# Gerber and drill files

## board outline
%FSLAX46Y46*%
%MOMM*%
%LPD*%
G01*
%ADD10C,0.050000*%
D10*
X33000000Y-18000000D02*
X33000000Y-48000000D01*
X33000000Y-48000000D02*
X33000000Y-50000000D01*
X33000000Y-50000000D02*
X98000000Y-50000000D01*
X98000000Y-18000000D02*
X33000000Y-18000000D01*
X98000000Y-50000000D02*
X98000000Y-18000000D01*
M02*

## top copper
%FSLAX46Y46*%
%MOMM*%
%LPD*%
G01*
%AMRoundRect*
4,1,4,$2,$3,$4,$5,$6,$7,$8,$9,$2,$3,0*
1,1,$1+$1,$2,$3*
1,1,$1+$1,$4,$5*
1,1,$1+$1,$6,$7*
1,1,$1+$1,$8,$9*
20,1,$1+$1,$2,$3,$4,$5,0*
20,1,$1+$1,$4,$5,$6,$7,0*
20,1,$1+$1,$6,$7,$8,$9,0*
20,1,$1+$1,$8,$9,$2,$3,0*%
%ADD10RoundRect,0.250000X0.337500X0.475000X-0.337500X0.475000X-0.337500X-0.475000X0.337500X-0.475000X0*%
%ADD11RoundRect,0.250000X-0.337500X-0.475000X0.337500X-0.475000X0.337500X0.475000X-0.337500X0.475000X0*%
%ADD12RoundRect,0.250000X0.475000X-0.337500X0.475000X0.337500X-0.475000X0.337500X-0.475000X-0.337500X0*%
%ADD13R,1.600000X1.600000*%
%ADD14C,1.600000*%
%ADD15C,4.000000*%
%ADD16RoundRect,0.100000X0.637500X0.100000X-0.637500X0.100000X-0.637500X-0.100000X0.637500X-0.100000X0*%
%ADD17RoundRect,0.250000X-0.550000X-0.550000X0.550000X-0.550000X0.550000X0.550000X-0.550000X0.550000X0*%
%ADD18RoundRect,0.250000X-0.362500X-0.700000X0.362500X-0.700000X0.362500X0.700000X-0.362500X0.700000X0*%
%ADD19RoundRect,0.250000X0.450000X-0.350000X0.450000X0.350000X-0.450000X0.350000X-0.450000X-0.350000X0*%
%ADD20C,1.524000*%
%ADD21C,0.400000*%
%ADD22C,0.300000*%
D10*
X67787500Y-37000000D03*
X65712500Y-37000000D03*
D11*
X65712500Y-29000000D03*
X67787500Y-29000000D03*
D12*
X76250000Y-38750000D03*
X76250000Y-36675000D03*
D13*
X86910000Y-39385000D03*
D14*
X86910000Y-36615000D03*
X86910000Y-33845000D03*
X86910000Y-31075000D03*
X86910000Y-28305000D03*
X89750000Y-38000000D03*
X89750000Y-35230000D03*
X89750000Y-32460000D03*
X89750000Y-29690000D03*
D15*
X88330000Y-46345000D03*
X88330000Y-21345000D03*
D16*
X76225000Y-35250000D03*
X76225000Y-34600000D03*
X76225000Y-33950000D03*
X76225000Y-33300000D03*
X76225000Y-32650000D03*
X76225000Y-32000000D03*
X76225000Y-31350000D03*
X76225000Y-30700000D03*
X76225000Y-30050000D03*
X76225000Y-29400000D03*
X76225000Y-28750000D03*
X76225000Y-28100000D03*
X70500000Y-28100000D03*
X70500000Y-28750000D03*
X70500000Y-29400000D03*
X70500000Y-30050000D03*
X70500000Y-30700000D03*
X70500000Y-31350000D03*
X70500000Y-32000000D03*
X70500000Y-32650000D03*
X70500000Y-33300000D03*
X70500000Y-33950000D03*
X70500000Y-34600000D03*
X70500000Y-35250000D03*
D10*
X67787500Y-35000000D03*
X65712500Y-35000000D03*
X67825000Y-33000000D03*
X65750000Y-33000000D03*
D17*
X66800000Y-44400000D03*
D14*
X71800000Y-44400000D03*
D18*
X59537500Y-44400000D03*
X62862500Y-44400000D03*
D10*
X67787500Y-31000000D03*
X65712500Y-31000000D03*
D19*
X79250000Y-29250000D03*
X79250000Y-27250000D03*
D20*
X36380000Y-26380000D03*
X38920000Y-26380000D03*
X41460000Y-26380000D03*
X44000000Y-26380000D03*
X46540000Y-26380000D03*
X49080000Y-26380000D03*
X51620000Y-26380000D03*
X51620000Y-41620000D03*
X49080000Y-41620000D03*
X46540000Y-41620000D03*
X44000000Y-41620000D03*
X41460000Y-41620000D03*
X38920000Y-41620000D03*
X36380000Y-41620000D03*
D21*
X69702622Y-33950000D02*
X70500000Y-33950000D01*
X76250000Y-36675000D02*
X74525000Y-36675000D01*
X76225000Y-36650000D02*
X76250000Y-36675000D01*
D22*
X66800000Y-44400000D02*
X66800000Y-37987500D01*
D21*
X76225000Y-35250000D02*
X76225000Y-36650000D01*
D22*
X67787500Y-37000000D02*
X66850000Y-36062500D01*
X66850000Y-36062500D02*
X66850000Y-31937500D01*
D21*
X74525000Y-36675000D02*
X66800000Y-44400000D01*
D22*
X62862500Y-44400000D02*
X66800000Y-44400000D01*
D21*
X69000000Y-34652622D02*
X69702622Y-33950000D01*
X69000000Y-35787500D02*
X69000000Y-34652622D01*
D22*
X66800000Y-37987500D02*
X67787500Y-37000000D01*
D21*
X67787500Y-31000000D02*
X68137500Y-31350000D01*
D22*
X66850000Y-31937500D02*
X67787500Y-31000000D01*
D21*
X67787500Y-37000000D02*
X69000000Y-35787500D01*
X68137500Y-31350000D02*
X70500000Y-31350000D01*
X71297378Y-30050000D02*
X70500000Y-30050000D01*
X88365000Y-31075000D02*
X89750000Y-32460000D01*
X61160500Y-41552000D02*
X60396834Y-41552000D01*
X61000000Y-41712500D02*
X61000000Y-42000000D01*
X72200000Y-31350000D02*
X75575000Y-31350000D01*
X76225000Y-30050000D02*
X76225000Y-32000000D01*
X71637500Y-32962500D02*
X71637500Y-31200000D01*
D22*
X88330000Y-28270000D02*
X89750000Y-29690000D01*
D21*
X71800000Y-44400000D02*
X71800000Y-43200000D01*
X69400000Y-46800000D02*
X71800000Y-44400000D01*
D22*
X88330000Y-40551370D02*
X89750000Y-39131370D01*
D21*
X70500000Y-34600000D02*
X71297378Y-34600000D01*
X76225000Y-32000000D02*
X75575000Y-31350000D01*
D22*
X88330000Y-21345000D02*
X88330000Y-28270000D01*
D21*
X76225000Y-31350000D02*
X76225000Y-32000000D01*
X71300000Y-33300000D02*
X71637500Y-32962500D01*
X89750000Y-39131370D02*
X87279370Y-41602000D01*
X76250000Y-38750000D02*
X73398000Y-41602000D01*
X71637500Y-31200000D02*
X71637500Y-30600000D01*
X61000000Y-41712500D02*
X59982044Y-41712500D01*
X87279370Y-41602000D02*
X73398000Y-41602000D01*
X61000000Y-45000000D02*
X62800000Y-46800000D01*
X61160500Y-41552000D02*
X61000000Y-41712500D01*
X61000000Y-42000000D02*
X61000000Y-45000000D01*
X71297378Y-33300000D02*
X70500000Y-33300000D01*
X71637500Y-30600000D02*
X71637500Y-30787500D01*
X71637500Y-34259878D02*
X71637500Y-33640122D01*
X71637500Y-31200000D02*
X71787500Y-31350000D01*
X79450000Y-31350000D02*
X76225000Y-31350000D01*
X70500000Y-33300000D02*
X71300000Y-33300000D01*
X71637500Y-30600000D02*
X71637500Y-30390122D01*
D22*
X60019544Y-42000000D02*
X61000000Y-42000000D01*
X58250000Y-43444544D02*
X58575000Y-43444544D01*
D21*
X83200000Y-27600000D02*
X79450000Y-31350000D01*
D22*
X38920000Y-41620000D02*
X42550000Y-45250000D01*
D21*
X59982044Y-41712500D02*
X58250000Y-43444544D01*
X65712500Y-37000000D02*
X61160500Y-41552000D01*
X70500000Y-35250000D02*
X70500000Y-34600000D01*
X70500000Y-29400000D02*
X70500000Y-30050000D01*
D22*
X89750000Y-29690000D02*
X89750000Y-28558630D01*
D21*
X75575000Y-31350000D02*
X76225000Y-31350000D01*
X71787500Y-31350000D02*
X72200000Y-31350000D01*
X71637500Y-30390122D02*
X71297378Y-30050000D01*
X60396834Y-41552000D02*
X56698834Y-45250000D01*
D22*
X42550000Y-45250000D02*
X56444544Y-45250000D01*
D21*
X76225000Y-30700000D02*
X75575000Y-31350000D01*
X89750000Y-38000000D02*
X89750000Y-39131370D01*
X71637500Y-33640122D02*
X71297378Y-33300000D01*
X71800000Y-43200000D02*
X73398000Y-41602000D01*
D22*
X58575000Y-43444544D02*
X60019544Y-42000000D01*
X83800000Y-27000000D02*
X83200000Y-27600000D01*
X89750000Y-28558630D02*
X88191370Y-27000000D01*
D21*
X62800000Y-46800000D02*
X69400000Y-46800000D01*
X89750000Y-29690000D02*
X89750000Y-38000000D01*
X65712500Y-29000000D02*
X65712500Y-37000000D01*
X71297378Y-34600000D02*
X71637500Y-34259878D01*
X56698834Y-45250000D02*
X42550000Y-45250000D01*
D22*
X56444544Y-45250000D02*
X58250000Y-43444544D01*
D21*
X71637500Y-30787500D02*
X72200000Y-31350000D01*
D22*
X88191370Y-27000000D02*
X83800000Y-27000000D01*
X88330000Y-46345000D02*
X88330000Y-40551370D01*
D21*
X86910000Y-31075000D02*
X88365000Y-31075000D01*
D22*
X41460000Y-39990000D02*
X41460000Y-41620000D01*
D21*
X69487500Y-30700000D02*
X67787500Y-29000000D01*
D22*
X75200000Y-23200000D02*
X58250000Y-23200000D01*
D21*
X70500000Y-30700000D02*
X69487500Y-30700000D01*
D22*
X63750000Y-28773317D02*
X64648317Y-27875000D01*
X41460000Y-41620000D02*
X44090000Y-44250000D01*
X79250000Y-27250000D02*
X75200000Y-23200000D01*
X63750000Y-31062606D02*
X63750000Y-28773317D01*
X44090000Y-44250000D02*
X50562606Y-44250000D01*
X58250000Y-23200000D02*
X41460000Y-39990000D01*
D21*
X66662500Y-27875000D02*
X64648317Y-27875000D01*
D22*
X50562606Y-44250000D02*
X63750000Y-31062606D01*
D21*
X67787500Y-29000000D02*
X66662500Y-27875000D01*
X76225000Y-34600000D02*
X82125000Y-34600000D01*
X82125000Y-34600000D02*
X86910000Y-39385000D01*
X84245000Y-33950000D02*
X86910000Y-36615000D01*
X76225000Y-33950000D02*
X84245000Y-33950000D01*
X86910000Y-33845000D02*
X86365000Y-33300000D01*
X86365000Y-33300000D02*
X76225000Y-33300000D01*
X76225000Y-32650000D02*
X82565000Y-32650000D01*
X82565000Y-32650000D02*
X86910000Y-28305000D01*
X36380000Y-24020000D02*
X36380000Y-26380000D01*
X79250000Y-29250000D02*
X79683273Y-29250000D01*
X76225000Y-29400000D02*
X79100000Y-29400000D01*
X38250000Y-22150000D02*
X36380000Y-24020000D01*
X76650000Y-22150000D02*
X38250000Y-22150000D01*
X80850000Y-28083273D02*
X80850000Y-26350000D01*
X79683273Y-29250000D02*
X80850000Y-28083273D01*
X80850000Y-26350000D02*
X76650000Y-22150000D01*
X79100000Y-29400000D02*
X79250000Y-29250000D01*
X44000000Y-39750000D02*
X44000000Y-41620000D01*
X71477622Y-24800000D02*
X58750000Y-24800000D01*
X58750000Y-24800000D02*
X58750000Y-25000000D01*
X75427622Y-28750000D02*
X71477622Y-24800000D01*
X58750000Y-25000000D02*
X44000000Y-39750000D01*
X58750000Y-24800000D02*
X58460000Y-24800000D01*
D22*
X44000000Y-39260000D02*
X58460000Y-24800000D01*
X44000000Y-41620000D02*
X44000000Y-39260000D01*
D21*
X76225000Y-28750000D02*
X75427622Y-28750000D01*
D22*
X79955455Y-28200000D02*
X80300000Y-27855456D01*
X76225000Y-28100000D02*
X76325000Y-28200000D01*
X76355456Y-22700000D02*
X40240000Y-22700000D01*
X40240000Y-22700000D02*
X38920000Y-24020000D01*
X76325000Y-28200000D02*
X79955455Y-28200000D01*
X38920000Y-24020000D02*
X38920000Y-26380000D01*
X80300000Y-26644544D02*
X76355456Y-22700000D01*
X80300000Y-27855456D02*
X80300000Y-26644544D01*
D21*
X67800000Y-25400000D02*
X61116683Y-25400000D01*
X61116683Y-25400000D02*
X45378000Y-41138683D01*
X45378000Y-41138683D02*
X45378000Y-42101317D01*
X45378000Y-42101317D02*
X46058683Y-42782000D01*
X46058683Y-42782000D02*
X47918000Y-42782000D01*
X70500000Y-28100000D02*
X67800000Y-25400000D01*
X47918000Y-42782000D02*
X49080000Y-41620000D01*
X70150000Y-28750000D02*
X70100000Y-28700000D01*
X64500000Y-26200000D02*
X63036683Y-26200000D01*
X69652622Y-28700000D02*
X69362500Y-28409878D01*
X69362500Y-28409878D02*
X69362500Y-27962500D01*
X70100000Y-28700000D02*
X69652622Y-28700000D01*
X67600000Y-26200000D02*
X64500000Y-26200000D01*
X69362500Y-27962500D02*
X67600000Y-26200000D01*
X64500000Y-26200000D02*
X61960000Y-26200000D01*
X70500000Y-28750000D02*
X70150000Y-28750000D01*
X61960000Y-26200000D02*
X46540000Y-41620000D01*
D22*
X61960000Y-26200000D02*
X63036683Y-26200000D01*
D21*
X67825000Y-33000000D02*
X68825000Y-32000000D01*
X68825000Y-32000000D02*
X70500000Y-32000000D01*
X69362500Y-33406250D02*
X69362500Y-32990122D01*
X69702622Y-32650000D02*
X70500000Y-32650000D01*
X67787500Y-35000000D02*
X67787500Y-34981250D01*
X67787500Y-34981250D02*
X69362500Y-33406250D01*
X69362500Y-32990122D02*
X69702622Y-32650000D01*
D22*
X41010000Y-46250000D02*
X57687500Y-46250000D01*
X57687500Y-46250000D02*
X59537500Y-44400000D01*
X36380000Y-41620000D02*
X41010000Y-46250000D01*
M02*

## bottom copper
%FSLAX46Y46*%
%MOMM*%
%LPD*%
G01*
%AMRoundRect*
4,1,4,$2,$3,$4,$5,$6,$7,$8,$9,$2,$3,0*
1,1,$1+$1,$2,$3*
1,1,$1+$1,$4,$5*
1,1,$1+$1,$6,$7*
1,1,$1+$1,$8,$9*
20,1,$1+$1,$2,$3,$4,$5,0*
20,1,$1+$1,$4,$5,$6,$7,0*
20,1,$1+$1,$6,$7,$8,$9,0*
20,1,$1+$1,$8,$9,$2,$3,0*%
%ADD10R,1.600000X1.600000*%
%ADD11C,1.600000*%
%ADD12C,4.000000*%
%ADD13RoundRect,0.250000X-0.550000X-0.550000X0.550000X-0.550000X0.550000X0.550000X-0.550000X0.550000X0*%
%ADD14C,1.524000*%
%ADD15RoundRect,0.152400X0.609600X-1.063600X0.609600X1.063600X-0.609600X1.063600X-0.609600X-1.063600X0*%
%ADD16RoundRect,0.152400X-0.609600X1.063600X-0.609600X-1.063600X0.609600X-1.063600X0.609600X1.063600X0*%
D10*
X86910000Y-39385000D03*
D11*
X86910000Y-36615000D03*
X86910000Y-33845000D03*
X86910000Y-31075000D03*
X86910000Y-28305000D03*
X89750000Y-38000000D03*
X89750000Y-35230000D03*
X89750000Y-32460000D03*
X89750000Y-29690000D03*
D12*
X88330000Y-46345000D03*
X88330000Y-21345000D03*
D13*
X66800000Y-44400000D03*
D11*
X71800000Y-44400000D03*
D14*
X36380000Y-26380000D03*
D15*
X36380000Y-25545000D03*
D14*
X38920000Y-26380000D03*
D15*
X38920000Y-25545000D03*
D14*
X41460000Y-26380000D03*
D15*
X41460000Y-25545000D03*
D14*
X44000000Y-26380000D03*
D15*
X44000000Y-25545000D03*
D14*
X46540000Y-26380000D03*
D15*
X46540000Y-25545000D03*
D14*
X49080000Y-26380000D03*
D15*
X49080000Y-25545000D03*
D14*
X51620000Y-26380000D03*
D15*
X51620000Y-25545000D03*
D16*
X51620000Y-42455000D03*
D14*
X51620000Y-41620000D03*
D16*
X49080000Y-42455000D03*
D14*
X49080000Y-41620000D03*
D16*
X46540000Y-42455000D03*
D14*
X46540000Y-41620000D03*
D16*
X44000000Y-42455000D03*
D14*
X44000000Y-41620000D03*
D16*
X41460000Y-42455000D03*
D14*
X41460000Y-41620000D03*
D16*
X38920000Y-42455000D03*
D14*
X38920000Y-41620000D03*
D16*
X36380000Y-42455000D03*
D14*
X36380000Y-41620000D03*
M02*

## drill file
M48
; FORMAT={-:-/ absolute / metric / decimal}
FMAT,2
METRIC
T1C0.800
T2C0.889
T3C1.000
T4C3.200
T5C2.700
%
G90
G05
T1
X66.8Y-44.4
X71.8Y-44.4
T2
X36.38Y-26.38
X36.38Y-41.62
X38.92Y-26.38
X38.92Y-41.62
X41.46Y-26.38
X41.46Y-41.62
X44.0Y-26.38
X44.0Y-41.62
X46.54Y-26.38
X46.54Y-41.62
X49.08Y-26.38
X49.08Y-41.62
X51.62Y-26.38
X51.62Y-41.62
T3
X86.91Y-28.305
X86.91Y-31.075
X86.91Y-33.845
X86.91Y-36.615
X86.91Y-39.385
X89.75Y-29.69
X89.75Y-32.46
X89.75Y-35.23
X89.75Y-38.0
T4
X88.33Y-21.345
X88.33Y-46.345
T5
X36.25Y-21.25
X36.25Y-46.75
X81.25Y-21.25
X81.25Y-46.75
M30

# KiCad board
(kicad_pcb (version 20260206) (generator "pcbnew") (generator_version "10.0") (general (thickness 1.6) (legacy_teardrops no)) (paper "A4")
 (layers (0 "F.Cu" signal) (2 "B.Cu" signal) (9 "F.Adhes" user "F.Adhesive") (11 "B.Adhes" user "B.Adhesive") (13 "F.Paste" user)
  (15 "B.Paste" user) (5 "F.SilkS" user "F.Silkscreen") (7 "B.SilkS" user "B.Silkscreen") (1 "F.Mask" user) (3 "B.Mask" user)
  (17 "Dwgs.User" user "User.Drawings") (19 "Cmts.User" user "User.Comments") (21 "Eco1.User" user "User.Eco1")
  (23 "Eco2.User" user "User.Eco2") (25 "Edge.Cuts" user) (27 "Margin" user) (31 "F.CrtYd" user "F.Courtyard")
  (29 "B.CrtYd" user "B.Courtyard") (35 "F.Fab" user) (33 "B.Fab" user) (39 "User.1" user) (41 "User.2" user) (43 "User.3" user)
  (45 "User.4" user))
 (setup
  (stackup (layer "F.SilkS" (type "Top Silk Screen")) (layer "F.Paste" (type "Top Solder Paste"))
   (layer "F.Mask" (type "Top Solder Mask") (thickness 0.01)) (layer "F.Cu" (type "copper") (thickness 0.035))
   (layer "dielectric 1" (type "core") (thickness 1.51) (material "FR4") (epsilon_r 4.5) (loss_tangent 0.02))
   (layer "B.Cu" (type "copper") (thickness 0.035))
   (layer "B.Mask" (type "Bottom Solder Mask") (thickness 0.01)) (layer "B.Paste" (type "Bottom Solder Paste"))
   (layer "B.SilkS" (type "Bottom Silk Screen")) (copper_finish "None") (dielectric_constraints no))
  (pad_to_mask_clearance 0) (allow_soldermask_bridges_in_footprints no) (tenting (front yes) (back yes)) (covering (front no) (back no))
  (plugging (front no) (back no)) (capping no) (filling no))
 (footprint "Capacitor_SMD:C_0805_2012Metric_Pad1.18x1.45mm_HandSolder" (layer "F.Cu") (at 66.75 37 180)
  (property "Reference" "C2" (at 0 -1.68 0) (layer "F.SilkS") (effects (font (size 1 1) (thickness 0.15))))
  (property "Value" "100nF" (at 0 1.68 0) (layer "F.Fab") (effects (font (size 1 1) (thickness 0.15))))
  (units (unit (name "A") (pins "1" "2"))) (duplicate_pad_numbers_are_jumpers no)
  (pad "1" smd roundrect (at -1.0375 0 180) (size 1.175 1.45) (layers "F.Cu" "F.Mask" "F.Paste") (roundrect_rratio 0.212766)
   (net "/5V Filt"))
  (pad "2" smd roundrect (at 1.0375 0 180) (size 1.175 1.45) (layers "F.Cu" "F.Mask" "F.Paste") (roundrect_rratio 0.212766) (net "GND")))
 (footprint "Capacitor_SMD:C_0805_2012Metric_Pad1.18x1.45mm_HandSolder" (layer "F.Cu") (at 66.75 29)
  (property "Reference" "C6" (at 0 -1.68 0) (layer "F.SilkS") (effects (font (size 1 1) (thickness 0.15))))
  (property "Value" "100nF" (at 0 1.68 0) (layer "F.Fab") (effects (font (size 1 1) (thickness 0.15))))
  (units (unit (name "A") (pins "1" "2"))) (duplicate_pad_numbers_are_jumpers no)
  (pad "1" smd roundrect (at -1.0375 0) (size 1.175 1.45) (layers "F.Cu" "F.Mask" "F.Paste") (roundrect_rratio 0.212766) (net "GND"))
  (pad "2" smd roundrect (at 1.0375 0) (size 1.175 1.45) (layers "F.Cu" "F.Mask" "F.Paste") (roundrect_rratio 0.212766) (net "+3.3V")))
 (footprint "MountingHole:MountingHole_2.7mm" (layer "F.Cu") (at 81.25 46.75)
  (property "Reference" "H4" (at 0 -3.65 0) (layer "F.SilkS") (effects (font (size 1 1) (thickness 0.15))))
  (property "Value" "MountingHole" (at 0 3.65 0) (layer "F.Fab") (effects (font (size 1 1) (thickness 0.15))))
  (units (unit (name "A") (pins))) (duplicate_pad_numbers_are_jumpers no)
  (pad "" np_thru_hole circle (at 0 0) (size 2.7 2.7) (drill 2.7) (layers "*.Cu" "*.Mask")))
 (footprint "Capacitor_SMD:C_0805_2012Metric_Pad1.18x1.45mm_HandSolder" (layer "F.Cu") (at 76.25 37.7125 90)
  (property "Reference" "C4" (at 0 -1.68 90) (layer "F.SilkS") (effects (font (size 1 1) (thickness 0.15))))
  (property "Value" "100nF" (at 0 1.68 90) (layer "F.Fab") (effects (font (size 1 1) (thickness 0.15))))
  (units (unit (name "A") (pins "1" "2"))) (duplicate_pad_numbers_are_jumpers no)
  (pad "1" smd roundrect (at -1.0375 0 90) (size 1.175 1.45) (layers "F.Cu" "F.Mask" "F.Paste") (roundrect_rratio 0.212766) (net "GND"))
  (pad "2" smd roundrect (at 1.0375 0 90) (size 1.175 1.45) (layers "F.Cu" "F.Mask" "F.Paste") (roundrect_rratio 0.212766) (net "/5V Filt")))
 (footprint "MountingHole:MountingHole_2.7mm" (layer "F.Cu") (at 81.25 21.25)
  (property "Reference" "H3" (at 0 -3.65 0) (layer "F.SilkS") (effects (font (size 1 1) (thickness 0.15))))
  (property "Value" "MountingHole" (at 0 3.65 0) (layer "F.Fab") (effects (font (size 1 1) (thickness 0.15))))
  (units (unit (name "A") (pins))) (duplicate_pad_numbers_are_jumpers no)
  (pad "" np_thru_hole circle (at 0 0) (size 2.7 2.7) (drill 2.7) (layers "*.Cu" "*.Mask")))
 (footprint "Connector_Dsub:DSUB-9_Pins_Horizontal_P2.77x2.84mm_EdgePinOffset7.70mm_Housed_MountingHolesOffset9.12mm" (layer "F.Cu")
  (at 86.91 39.385 90)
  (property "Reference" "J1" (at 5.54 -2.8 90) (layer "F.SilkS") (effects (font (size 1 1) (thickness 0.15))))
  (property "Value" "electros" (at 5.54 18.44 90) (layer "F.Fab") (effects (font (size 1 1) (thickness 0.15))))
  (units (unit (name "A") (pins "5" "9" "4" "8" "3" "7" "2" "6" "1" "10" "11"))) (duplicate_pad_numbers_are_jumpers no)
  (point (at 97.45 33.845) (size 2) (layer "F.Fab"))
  (pad "1" thru_hole rect (at 0 0 90) (size 1.6 1.6) (drill 1) (layers "*.Cu" "*.Mask") (remove_unused_layers no) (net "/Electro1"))
  (pad "2" thru_hole circle (at 2.77 0 90) (size 1.6 1.6) (drill 1) (layers "*.Cu" "*.Mask") (remove_unused_layers no) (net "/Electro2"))
  (pad "3" thru_hole circle (at 5.54 0 90) (size 1.6 1.6) (drill 1) (layers "*.Cu" "*.Mask") (remove_unused_layers no) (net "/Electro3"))
  (pad "4" thru_hole circle (at 8.31 0 90) (size 1.6 1.6) (drill 1) (layers "*.Cu" "*.Mask") (remove_unused_layers no) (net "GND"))
  (pad "5" thru_hole circle (at 11.08 0 90) (size 1.6 1.6) (drill 1) (layers "*.Cu" "*.Mask") (remove_unused_layers no) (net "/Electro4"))
  (pad "6" thru_hole circle (at 1.385 2.84 90) (size 1.6 1.6) (drill 1) (layers "*.Cu" "*.Mask") (remove_unused_layers no) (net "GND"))
  (pad "7" thru_hole circle (at 4.155 2.84 90) (size 1.6 1.6) (drill 1) (layers "*.Cu" "*.Mask") (remove_unused_layers no) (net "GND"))
  (pad "8" thru_hole circle (at 6.925 2.84 90) (size 1.6 1.6) (drill 1) (layers "*.Cu" "*.Mask") (remove_unused_layers no) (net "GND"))
  (pad "9" thru_hole circle (at 9.695 2.84 90) (size 1.6 1.6) (drill 1) (layers "*.Cu" "*.Mask") (remove_unused_layers no) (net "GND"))
  (pad "SH" thru_hole circle (at -6.96 1.42 90) (size 4 4) (drill 3.2) (layers "*.Cu" "*.Mask") (remove_unused_layers no) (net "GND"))
  (pad "SH" thru_hole circle (at 18.04 1.42 90) (size 4 4) (drill 3.2) (layers "*.Cu" "*.Mask") (remove_unused_layers no) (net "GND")))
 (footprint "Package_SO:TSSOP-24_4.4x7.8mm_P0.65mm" (layer "F.Cu") (at 73.3625 31.675 180)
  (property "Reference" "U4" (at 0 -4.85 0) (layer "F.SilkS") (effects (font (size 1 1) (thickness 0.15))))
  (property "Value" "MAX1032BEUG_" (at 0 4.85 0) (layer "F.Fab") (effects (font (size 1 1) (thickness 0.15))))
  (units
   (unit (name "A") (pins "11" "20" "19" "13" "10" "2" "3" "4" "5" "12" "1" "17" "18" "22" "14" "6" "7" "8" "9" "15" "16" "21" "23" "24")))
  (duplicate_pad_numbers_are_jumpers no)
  (pad "1" smd roundrect (at -2.8625 -3.575 180) (size 1.475 0.4) (layers "F.Cu" "F.Mask" "F.Paste") (roundrect_rratio 0.25)
   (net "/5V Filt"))
  (pad "2" smd roundrect (at -2.8625 -2.925 180) (size 1.475 0.4) (layers "F.Cu" "F.Mask" "F.Paste") (roundrect_rratio 0.25)
   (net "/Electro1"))
  (pad "3" smd roundrect (at -2.8625 -2.275 180) (size 1.475 0.4) (layers "F.Cu" "F.Mask" "F.Paste") (roundrect_rratio 0.25)
   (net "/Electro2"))
  (pad "4" smd roundrect (at -2.8625 -1.625 180) (size 1.475 0.4) (layers "F.Cu" "F.Mask" "F.Paste") (roundrect_rratio 0.25)
   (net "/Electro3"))
  (pad "5" smd roundrect (at -2.8625 -0.975 180) (size 1.475 0.4) (layers "F.Cu" "F.Mask" "F.Paste") (roundrect_rratio 0.25)
   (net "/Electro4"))
  (pad "6" smd roundrect (at -2.8625 -0.325 180) (size 1.475 0.4) (layers "F.Cu" "F.Mask" "F.Paste") (roundrect_rratio 0.25) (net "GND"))
  (pad "7" smd roundrect (at -2.8625 0.325 180) (size 1.475 0.4) (layers "F.Cu" "F.Mask" "F.Paste") (roundrect_rratio 0.25) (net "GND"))
  (pad "8" smd roundrect (at -2.8625 0.975 180) (size 1.475 0.4) (layers "F.Cu" "F.Mask" "F.Paste") (roundrect_rratio 0.25) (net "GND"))
  (pad "9" smd roundrect (at -2.8625 1.625 180) (size 1.475 0.4) (layers "F.Cu" "F.Mask" "F.Paste") (roundrect_rratio 0.25) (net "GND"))
  (pad "10" smd roundrect (at -2.8625 2.275 180) (size 1.475 0.4) (layers "F.Cu" "F.Mask" "F.Paste") (roundrect_rratio 0.25) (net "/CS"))
  (pad "11" smd roundrect (at -2.8625 2.925 180) (size 1.475 0.4) (layers "F.Cu" "F.Mask" "F.Paste") (roundrect_rratio 0.25) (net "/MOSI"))
  (pad "12" smd roundrect (at -2.8625 3.575 180) (size 1.475 0.4) (layers "F.Cu" "F.Mask" "F.Paste") (roundrect_rratio 0.25) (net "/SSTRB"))
  (pad "13" smd roundrect (at 2.8625 3.575 180) (size 1.475 0.4) (layers "F.Cu" "F.Mask" "F.Paste") (roundrect_rratio 0.25) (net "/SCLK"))
  (pad "14" smd roundrect (at 2.8625 2.925 180) (size 1.475 0.4) (layers "F.Cu" "F.Mask" "F.Paste") (roundrect_rratio 0.25) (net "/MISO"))
  (pad "15" smd roundrect (at 2.8625 2.275 180) (size 1.475 0.4) (layers "F.Cu" "F.Mask" "F.Paste") (roundrect_rratio 0.25) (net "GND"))
  (pad "16" smd roundrect (at 2.8625 1.625 180) (size 1.475 0.4) (layers "F.Cu" "F.Mask" "F.Paste") (roundrect_rratio 0.25) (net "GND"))
  (pad "17" smd roundrect (at 2.8625 0.975 180) (size 1.475 0.4) (layers "F.Cu" "F.Mask" "F.Paste") (roundrect_rratio 0.25) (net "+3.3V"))
  (pad "18" smd roundrect (at 2.8625 0.325 180) (size 1.475 0.4) (layers "F.Cu" "F.Mask" "F.Paste") (roundrect_rratio 0.25) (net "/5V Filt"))
  (pad "19" smd roundrect (at 2.8625 -0.325 180) (size 1.475 0.4) (layers "F.Cu" "F.Mask" "F.Paste") (roundrect_rratio 0.25)
   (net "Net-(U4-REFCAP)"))
  (pad "20" smd roundrect (at 2.8625 -0.975 180) (size 1.475 0.4) (layers "F.Cu" "F.Mask" "F.Paste") (roundrect_rratio 0.25)
   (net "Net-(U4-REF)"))
  (pad "21" smd roundrect (at 2.8625 -1.625 180) (size 1.475 0.4) (layers "F.Cu" "F.Mask" "F.Paste") (roundrect_rratio 0.25) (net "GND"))
  (pad "22" smd roundrect (at 2.8625 -2.275 180) (size 1.475 0.4) (layers "F.Cu" "F.Mask" "F.Paste") (roundrect_rratio 0.25)
   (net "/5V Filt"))
  (pad "23" smd roundrect (at 2.8625 -2.925 180) (size 1.475 0.4) (layers "F.Cu" "F.Mask" "F.Paste") (roundrect_rratio 0.25) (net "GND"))
  (pad "24" smd roundrect (at 2.8625 -3.575 180) (size 1.475 0.4) (layers "F.Cu" "F.Mask" "F.Paste") (roundrect_rratio 0.25) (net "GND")))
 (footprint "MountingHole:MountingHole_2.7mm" (layer "F.Cu") (at 36.25 46.75)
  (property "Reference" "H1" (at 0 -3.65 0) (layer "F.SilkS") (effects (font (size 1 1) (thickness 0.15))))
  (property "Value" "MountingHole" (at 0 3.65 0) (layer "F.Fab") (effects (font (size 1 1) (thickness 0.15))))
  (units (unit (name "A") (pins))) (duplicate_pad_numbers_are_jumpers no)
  (pad "" np_thru_hole circle (at 0 0) (size 2.7 2.7) (drill 2.7) (layers "*.Cu" "*.Mask")))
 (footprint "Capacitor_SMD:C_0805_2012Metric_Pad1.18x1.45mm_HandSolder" (layer "F.Cu") (at 66.75 35 180)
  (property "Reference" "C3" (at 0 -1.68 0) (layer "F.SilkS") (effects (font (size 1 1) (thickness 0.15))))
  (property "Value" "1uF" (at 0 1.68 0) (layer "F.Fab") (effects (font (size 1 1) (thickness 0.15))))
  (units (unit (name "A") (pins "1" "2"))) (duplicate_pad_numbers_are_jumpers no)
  (pad "1" smd roundrect (at -1.0375 0 180) (size 1.175 1.45) (layers "F.Cu" "F.Mask" "F.Paste") (roundrect_rratio 0.212766)
   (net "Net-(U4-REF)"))
  (pad "2" smd roundrect (at 1.0375 0 180) (size 1.175 1.45) (layers "F.Cu" "F.Mask" "F.Paste") (roundrect_rratio 0.212766) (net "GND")))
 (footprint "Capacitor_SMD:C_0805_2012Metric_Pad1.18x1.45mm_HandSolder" (layer "F.Cu") (at 66.7875 33 180)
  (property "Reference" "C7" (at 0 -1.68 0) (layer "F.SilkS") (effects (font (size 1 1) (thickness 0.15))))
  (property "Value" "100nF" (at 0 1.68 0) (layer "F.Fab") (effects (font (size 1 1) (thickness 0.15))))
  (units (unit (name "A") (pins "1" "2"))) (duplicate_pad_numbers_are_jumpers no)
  (pad "1" smd roundrect (at -1.0375 0 180) (size 1.175 1.45) (layers "F.Cu" "F.Mask" "F.Paste") (roundrect_rratio 0.212766)
   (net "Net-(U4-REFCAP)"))
  (pad "2" smd roundrect (at 1.0375 0 180) (size 1.175 1.45) (layers "F.Cu" "F.Mask" "F.Paste") (roundrect_rratio 0.212766) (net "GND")))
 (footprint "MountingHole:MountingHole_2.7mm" (layer "F.Cu") (at 36.25 21.25)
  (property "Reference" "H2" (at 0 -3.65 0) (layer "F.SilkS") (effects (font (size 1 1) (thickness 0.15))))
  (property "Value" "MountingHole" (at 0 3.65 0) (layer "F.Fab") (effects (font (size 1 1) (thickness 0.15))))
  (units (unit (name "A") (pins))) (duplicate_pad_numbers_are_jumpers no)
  (pad "" np_thru_hole circle (at 0 0) (size 2.7 2.7) (drill 2.7) (layers "*.Cu" "*.Mask")))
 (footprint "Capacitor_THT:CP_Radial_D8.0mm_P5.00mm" (layer "F.Cu") (at 66.8 44.4)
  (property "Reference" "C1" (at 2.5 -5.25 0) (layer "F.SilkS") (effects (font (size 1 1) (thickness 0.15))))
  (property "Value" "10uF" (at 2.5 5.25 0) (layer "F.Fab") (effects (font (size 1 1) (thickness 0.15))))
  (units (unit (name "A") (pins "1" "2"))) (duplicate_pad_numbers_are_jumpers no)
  (pad "1" thru_hole roundrect (at 0 0) (size 1.6 1.6) (drill 0.8) (layers "*.Cu" "*.Mask") (remove_unused_layers no)
   (roundrect_rratio 0.15625) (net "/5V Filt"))
  (pad "2" thru_hole circle (at 5 0) (size 1.6 1.6) (drill 0.8) (layers "*.Cu" "*.Mask") (remove_unused_layers no) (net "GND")))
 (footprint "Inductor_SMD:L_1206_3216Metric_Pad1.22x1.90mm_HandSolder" (layer "F.Cu") (at 61.2 44.4)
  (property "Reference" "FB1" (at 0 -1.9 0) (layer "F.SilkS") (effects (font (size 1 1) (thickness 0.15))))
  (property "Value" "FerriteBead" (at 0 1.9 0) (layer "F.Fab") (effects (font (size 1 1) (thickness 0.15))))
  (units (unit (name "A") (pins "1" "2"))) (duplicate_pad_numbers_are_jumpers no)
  (pad "1" smd roundrect (at -1.6625 0) (size 1.225 1.9) (layers "F.Cu" "F.Mask" "F.Paste") (roundrect_rratio 0.204082) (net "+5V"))
  (pad "2" smd roundrect (at 1.6625 0) (size 1.225 1.9) (layers "F.Cu" "F.Mask" "F.Paste") (roundrect_rratio 0.204082) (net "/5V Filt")))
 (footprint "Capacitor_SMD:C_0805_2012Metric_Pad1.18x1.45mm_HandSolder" (layer "F.Cu") (at 66.75 31 180)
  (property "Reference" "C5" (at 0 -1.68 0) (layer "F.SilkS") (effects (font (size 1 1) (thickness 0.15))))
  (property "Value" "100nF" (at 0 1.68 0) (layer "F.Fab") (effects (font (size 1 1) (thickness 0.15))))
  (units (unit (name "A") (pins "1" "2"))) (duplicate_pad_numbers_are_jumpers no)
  (pad "1" smd roundrect (at -1.0375 0 180) (size 1.175 1.45) (layers "F.Cu" "F.Mask" "F.Paste") (roundrect_rratio 0.212766)
   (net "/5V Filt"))
  (pad "2" smd roundrect (at 1.0375 0 180) (size 1.175 1.45) (layers "F.Cu" "F.Mask" "F.Paste") (roundrect_rratio 0.212766) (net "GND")))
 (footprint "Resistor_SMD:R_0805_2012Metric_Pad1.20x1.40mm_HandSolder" (layer "F.Cu") (at 79.25 28.25 90)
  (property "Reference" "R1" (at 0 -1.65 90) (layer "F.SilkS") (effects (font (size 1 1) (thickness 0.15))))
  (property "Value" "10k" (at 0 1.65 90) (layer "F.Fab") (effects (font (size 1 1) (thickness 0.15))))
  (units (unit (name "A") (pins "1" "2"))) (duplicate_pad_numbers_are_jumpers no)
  (pad "1" smd roundrect (at -1 0 90) (size 1.2 1.4) (layers "F.Cu" "F.Mask" "F.Paste") (roundrect_rratio 0.208333) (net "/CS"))
  (pad "2" smd roundrect (at 1 0 90) (size 1.2 1.4) (layers "F.Cu" "F.Mask" "F.Paste") (roundrect_rratio 0.208333) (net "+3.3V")))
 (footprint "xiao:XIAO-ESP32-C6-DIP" (layer "B.Cu") (at 44 34 180)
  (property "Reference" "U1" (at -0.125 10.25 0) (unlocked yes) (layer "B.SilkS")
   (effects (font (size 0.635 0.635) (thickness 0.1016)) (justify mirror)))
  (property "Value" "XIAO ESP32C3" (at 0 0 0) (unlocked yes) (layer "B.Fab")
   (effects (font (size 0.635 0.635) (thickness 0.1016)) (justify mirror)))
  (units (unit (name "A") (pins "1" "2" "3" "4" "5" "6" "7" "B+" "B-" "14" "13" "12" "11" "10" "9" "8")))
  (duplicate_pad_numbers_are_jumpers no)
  (pad "1" thru_hole circle (at 7.62 7.62 90) (size 1.524 1.524) (drill 0.889) (layers "*.Cu" "*.Mask") (remove_unused_layers no)
   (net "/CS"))
  (pad "1" smd roundrect (at 7.62 8.455 90) (size 2.432 1.524) (layers "B.Cu" "B.Mask") (roundrect_rratio 0.1) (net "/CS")
   (thermal_bridge_angle 45))
  (pad "2" thru_hole circle (at 5.08 7.62 90) (size 1.524 1.524) (drill 0.889) (layers "*.Cu" "*.Mask") (remove_unused_layers no)
   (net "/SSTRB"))
  (pad "2" smd roundrect (at 5.08 8.455 90) (size 2.432 1.524) (layers "B.Cu" "B.Mask") (roundrect_rratio 0.1) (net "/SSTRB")
   (thermal_bridge_angle 45))
  (pad "3" thru_hole circle (at 2.54 7.62 90) (size 1.524 1.524) (drill 0.889) (layers "*.Cu" "*.Mask") (remove_unused_layers no)
   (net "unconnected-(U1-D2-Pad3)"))
  (pad "3" smd roundrect (at 2.54 8.455 90) (size 2.432 1.524) (layers "B.Cu" "B.Mask") (roundrect_rratio 0.1)
   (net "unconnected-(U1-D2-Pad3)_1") (thermal_bridge_angle 45))
  (pad "4" thru_hole circle (at 0 7.62 90) (size 1.524 1.524) (drill 0.889) (layers "*.Cu" "*.Mask") (remove_unused_layers no)
   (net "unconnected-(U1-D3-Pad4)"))
  (pad "4" smd roundrect (at 0 8.455 90) (size 2.432 1.524) (layers "B.Cu" "B.Mask") (roundrect_rratio 0.1)
   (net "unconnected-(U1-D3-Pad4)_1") (thermal_bridge_angle 45))
  (pad "5" thru_hole circle (at -2.54 7.62 90) (size 1.524 1.524) (drill 0.889) (layers "*.Cu" "*.Mask") (remove_unused_layers no)
   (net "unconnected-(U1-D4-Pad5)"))
  (pad "5" smd roundrect (at -2.54 8.455 90) (size 2.432 1.524) (layers "B.Cu" "B.Mask") (roundrect_rratio 0.1)
   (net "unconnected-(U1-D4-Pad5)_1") (thermal_bridge_angle 45))
  (pad "6" thru_hole circle (at -5.08 7.62 90) (size 1.524 1.524) (drill 0.889) (layers "*.Cu" "*.Mask") (remove_unused_layers no)
   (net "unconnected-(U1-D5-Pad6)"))
  (pad "6" smd roundrect (at -5.08 8.455 90) (size 2.432 1.524) (layers "B.Cu" "B.Mask") (roundrect_rratio 0.1)
   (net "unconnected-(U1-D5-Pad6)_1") (thermal_bridge_angle 45))
  (pad "7" thru_hole circle (at -7.62 7.62 90) (size 1.524 1.524) (drill 0.889) (layers "*.Cu" "*.Mask") (remove_unused_layers no)
   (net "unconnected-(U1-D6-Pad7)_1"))
  (pad "7" smd roundrect (at -7.62 8.455 90) (size 2.432 1.524) (layers "B.Cu" "B.Mask") (roundrect_rratio 0.1)
   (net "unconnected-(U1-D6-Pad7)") (thermal_bridge_angle 45))
  (pad "8" smd roundrect (at -7.62 -8.455 270) (size 2.432 1.524) (layers "B.Cu" "B.Mask") (roundrect_rratio 0.1)
   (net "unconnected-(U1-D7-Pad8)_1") (thermal_bridge_angle 45))
  (pad "8" thru_hole circle (at -7.62 -7.62 270) (size 1.524 1.524) (drill 0.889) (layers "*.Cu" "*.Mask") (remove_unused_layers no)
   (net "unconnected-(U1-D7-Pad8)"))
  (pad "9" smd roundrect (at -5.08 -8.455 270) (size 2.432 1.524) (layers "B.Cu" "B.Mask") (roundrect_rratio 0.1) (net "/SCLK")
   (thermal_bridge_angle 45))
  (pad "9" thru_hole circle (at -5.08 -7.62 270) (size 1.524 1.524) (drill 0.889) (layers "*.Cu" "*.Mask") (remove_unused_layers no)
   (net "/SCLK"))
  (pad "10" smd roundrect (at -2.54 -8.455 270) (size 2.432 1.524) (layers "B.Cu" "B.Mask") (roundrect_rratio 0.1) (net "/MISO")
   (thermal_bridge_angle 45))
  (pad "10" thru_hole circle (at -2.54 -7.62 270) (size 1.524 1.524) (drill 0.889) (layers "*.Cu" "*.Mask") (remove_unused_layers no)
   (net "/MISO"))
  (pad "11" smd roundrect (at 0 -8.455 270) (size 2.432 1.524) (layers "B.Cu" "B.Mask") (roundrect_rratio 0.1) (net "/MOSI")
   (thermal_bridge_angle 45))
  (pad "11" thru_hole circle (at 0 -7.62 270) (size 1.524 1.524) (drill 0.889) (layers "*.Cu" "*.Mask") (remove_unused_layers no)
   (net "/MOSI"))
  (pad "12" smd roundrect (at 2.54 -8.455 270) (size 2.432 1.524) (layers "B.Cu" "B.Mask") (roundrect_rratio 0.1) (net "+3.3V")
   (thermal_bridge_angle 45))
  (pad "12" thru_hole circle (at 2.54 -7.62 270) (size 1.524 1.524) (drill 0.889) (layers "*.Cu" "*.Mask") (remove_unused_layers no)
   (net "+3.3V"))
  (pad "13" smd roundrect (at 5.08 -8.455 270) (size 2.432 1.524) (layers "B.Cu" "B.Mask") (roundrect_rratio 0.1) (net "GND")
   (thermal_bridge_angle 45))
  (pad "13" thru_hole circle (at 5.08 -7.62 270) (size 1.524 1.524) (drill 0.889) (layers "*.Cu" "*.Mask") (remove_unused_layers no)
   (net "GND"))
  (pad "14" smd roundrect (at 7.62 -8.455 270) (size 2.432 1.524) (layers "B.Cu" "B.Mask") (roundrect_rratio 0.1) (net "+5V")
   (thermal_bridge_angle 45))
  (pad "14" thru_hole circle (at 7.62 -7.62 270) (size 1.524 1.524) (drill 0.889) (layers "*.Cu" "*.Mask") (remove_unused_layers no)
   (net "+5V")))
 (gr_line (start 33 18) (end 33 48) (stroke (width 0.05) (type default)) (layer "Edge.Cuts"))
 (gr_line (start 33 48) (end 33 50) (stroke (width 0.05) (type default)) (layer "Edge.Cuts"))
 (gr_line (start 33 50) (end 98 50) (stroke (width 0.05) (type default)) (layer "Edge.Cuts"))
 (gr_line (start 98 18) (end 33 18) (stroke (width 0.05) (type default)) (layer "Edge.Cuts"))
 (gr_line (start 98 50) (end 98 18) (stroke (width 0.05) (type default)) (layer "Edge.Cuts"))
 (segment (start 69.702622 33.95) (end 70.5 33.95) (width 0.4) (layer "F.Cu") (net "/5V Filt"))
 (segment (start 76.25 36.675) (end 74.525 36.675) (width 0.4) (layer "F.Cu") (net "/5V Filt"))
 (segment (start 76.225 36.65) (end 76.25 36.675) (width 0.4) (layer "F.Cu") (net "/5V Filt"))
 (segment (start 66.8 44.4) (end 66.8 37.9875) (width 0.3) (layer "F.Cu") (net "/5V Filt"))
 (segment (start 76.225 35.25) (end 76.225 36.65) (width 0.4) (layer "F.Cu") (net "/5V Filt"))
 (segment (start 67.7875 37) (end 66.85 36.0625) (width 0.3) (layer "F.Cu") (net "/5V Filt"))
 (segment (start 66.85 36.0625) (end 66.85 31.9375) (width 0.3) (layer "F.Cu") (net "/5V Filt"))
 (segment (start 74.525 36.675) (end 66.8 44.4) (width 0.4) (layer "F.Cu") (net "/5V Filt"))
 (segment (start 62.8625 44.4) (end 66.8 44.4) (width 0.3) (layer "F.Cu") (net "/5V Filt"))
 (segment (start 69 34.652622) (end 69.702622 33.95) (width 0.4) (layer "F.Cu") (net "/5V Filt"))
 (segment (start 69 35.7875) (end 69 34.652622) (width 0.4) (layer "F.Cu") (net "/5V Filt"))
 (segment (start 66.8 37.9875) (end 67.7875 37) (width 0.3) (layer "F.Cu") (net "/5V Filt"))
 (segment (start 67.7875 31) (end 68.1375 31.35) (width 0.4) (layer "F.Cu") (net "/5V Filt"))
 (segment (start 66.85 31.9375) (end 67.7875 31) (width 0.3) (layer "F.Cu") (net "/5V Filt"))
 (segment (start 67.7875 37) (end 69 35.7875) (width 0.4) (layer "F.Cu") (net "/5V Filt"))
 (segment (start 68.1375 31.35) (end 70.5 31.35) (width 0.4) (layer "F.Cu") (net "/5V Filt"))
 (segment (start 71.297378 30.05) (end 70.5 30.05) (width 0.4) (layer "F.Cu") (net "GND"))
 (segment (start 88.365 31.075) (end 89.75 32.46) (width 0.4) (layer "F.Cu") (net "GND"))
 (segment (start 61.1605 41.552) (end 60.396834 41.552) (width 0.4) (layer "F.Cu") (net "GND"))
 (segment (start 61 41.7125) (end 61 42) (width 0.4) (layer "F.Cu") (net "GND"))
 (segment (start 72.2 31.35) (end 75.575 31.35) (width 0.4) (layer "F.Cu") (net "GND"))
 (segment (start 76.225 30.05) (end 76.225 32) (width 0.4) (layer "F.Cu") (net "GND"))
 (segment (start 71.6375 32.9625) (end 71.6375 31.2) (width 0.4) (layer "F.Cu") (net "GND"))
 (segment (start 88.33 28.27) (end 89.75 29.69) (width 0.3) (layer "F.Cu") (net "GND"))
 (segment (start 71.8 44.4) (end 71.8 43.2) (width 0.4) (layer "F.Cu") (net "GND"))
 (segment (start 69.4 46.8) (end 71.8 44.4) (width 0.4) (layer "F.Cu") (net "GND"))
 (segment (start 88.33 40.55137) (end 89.75 39.13137) (width 0.3) (layer "F.Cu") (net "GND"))
 (segment (start 70.5 34.6) (end 71.297378 34.6) (width 0.4) (layer "F.Cu") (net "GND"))
 (segment (start 76.225 32) (end 75.575 31.35) (width 0.4) (layer "F.Cu") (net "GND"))
 (segment (start 88.33 21.345) (end 88.33 28.27) (width 0.3) (layer "F.Cu") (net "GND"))
 (segment (start 76.225 31.35) (end 76.225 32) (width 0.4) (layer "F.Cu") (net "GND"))
 (segment (start 71.3 33.3) (end 71.6375 32.9625) (width 0.4) (layer "F.Cu") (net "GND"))
 (segment (start 89.75 39.13137) (end 87.27937 41.602) (width 0.4) (layer "F.Cu") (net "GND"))
 (segment (start 76.25 38.75) (end 73.398 41.602) (width 0.4) (layer "F.Cu") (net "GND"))
 (segment (start 71.6375 31.2) (end 71.6375 30.6) (width 0.4) (layer "F.Cu") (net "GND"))
 (segment (start 61 41.7125) (end 59.982044 41.7125) (width 0.4) (layer "F.Cu") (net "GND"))
 (segment (start 87.27937 41.602) (end 73.398 41.602) (width 0.4) (layer "F.Cu") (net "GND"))
 (segment (start 61 45) (end 62.8 46.8) (width 0.4) (layer "F.Cu") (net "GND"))
 (segment (start 61.1605 41.552) (end 61 41.7125) (width 0.4) (layer "F.Cu") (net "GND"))
 (segment (start 61 42) (end 61 45) (width 0.4) (layer "F.Cu") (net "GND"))
 (segment (start 71.297378 33.3) (end 70.5 33.3) (width 0.4) (layer "F.Cu") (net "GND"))
 (segment (start 71.6375 30.6) (end 71.6375 30.7875) (width 0.4) (layer "F.Cu") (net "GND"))
 (segment (start 71.6375 34.259878) (end 71.6375 33.640122) (width 0.4) (layer "F.Cu") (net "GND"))
 (segment (start 71.6375 31.2) (end 71.7875 31.35) (width 0.4) (layer "F.Cu") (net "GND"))
 (segment (start 79.45 31.35) (end 76.225 31.35) (width 0.4) (layer "F.Cu") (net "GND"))
 (segment (start 70.5 33.3) (end 71.3 33.3) (width 0.4) (layer "F.Cu") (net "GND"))
 (segment (start 71.6375 30.6) (end 71.6375 30.390122) (width 0.4) (layer "F.Cu") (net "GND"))
 (segment (start 60.019544 42) (end 61 42) (width 0.3) (layer "F.Cu") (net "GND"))
 (segment (start 58.25 43.444544) (end 58.575 43.444544) (width 0.3) (layer "F.Cu") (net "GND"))
 (segment (start 83.2 27.6) (end 79.45 31.35) (width 0.4) (layer "F.Cu") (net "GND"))
 (segment (start 38.92 41.62) (end 42.55 45.25) (width 0.3) (layer "F.Cu") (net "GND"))
 (segment (start 59.982044 41.7125) (end 58.25 43.444544) (width 0.4) (layer "F.Cu") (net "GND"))
 (segment (start 65.7125 37) (end 61.1605 41.552) (width 0.4) (layer "F.Cu") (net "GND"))
 (segment (start 70.5 35.25) (end 70.5 34.6) (width 0.4) (layer "F.Cu") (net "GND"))
 (segment (start 70.5 29.4) (end 70.5 30.05) (width 0.4) (layer "F.Cu") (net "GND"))
 (segment (start 89.75 29.69) (end 89.75 28.55863) (width 0.3) (layer "F.Cu") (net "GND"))
 (segment (start 75.575 31.35) (end 76.225 31.35) (width 0.4) (layer "F.Cu") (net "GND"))
 (segment (start 71.7875 31.35) (end 72.2 31.35) (width 0.4) (layer "F.Cu") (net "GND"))
 (segment (start 71.6375 30.390122) (end 71.297378 30.05) (width 0.4) (layer "F.Cu") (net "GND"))
 (segment (start 60.396834 41.552) (end 56.698834 45.25) (width 0.4) (layer "F.Cu") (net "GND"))
 (segment (start 42.55 45.25) (end 56.444544 45.25) (width 0.3) (layer "F.Cu") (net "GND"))
 (segment (start 76.225 30.7) (end 75.575 31.35) (width 0.4) (layer "F.Cu") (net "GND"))
 (segment (start 89.75 38) (end 89.75 39.13137) (width 0.4) (layer "F.Cu") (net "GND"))
 (segment (start 71.6375 33.640122) (end 71.297378 33.3) (width 0.4) (layer "F.Cu") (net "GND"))
 (segment (start 71.8 43.2) (end 73.398 41.602) (width 0.4) (layer "F.Cu") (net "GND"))
 (segment (start 58.575 43.444544) (end 60.019544 42) (width 0.3) (layer "F.Cu") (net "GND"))
 (segment (start 83.8 27) (end 83.2 27.6) (width 0.3) (layer "F.Cu") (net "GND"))
 (segment (start 89.75 28.55863) (end 88.19137 27) (width 0.3) (layer "F.Cu") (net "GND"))
 (segment (start 62.8 46.8) (end 69.4 46.8) (width 0.4) (layer "F.Cu") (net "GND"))
 (segment (start 89.75 29.69) (end 89.75 38) (width 0.4) (layer "F.Cu") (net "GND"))
 (segment (start 65.7125 29) (end 65.7125 37) (width 0.4) (layer "F.Cu") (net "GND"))
 (segment (start 71.297378 34.6) (end 71.6375 34.259878) (width 0.4) (layer "F.Cu") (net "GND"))
 (segment (start 56.698834 45.25) (end 42.55 45.25) (width 0.4) (layer "F.Cu") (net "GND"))
 (segment (start 56.444544 45.25) (end 58.25 43.444544) (width 0.3) (layer "F.Cu") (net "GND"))
 (segment (start 71.6375 30.7875) (end 72.2 31.35) (width 0.4) (layer "F.Cu") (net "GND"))
 (segment (start 88.19137 27) (end 83.8 27) (width 0.3) (layer "F.Cu") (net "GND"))
 (segment (start 88.33 46.345) (end 88.33 40.55137) (width 0.3) (layer "F.Cu") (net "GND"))
 (segment (start 86.91 31.075) (end 88.365 31.075) (width 0.4) (layer "F.Cu") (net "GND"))
 (segment (start 41.46 39.99) (end 41.46 41.62) (width 0.3) (layer "F.Cu") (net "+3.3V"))
 (segment (start 69.4875 30.7) (end 67.7875 29) (width 0.4) (layer "F.Cu") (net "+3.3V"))
 (segment (start 75.2 23.2) (end 58.25 23.2) (width 0.3) (layer "F.Cu") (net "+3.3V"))
 (segment (start 70.5 30.7) (end 69.4875 30.7) (width 0.4) (layer "F.Cu") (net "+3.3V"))
 (segment (start 63.75 28.773317) (end 64.648317 27.875) (width 0.3) (layer "F.Cu") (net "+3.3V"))
 (segment (start 41.46 41.62) (end 44.09 44.25) (width 0.3) (layer "F.Cu") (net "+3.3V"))
 (segment (start 79.25 27.25) (end 75.2 23.2) (width 0.3) (layer "F.Cu") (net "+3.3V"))
 (segment (start 63.75 31.062606) (end 63.75 28.773317) (width 0.3) (layer "F.Cu") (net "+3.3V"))
 (segment (start 44.09 44.25) (end 50.562606 44.25) (width 0.3) (layer "F.Cu") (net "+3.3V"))
 (segment (start 58.25 23.2) (end 41.46 39.99) (width 0.3) (layer "F.Cu") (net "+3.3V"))
 (segment (start 66.6625 27.875) (end 64.648317 27.875) (width 0.4) (layer "F.Cu") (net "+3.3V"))
 (segment (start 50.562606 44.25) (end 63.75 31.062606) (width 0.3) (layer "F.Cu") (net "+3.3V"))
 (segment (start 67.7875 29) (end 66.6625 27.875) (width 0.4) (layer "F.Cu") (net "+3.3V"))
 (segment (start 76.225 34.6) (end 82.125 34.6) (width 0.4) (layer "F.Cu") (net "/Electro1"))
 (segment (start 82.125 34.6) (end 86.91 39.385) (width 0.4) (layer "F.Cu") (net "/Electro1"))
 (segment (start 84.245 33.95) (end 86.91 36.615) (width 0.4) (layer "F.Cu") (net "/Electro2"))
 (segment (start 76.225 33.95) (end 84.245 33.95) (width 0.4) (layer "F.Cu") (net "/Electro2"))
 (segment (start 86.91 33.845) (end 86.365 33.3) (width 0.4) (layer "F.Cu") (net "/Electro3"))
 (segment (start 86.365 33.3) (end 76.225 33.3) (width 0.4) (layer "F.Cu") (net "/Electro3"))
 (segment (start 76.225 32.65) (end 82.565 32.65) (width 0.4) (layer "F.Cu") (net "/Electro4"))
 (segment (start 82.565 32.65) (end 86.91 28.305) (width 0.4) (layer "F.Cu") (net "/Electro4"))
 (segment (start 36.38 24.02) (end 36.38 26.38) (width 0.4) (layer "F.Cu") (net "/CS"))
 (segment (start 79.25 29.25) (end 79.683273 29.25) (width 0.4) (layer "F.Cu") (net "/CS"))
 (segment (start 76.225 29.4) (end 79.1 29.4) (width 0.4) (layer "F.Cu") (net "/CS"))
 (segment (start 38.25 22.15) (end 36.38 24.02) (width 0.4) (layer "F.Cu") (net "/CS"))
 (segment (start 76.65 22.15) (end 38.25 22.15) (width 0.4) (layer "F.Cu") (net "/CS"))
 (segment (start 80.85 28.083273) (end 80.85 26.35) (width 0.4) (layer "F.Cu") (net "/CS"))
 (segment (start 79.683273 29.25) (end 80.85 28.083273) (width 0.4) (layer "F.Cu") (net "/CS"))
 (segment (start 80.85 26.35) (end 76.65 22.15) (width 0.4) (layer "F.Cu") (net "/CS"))
 (segment (start 79.1 29.4) (end 79.25 29.25) (width 0.4) (layer "F.Cu") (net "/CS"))
 (segment (start 44 39.75) (end 44 41.62) (width 0.4) (layer "F.Cu") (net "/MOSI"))
 (segment (start 71.477622 24.8) (end 58.75 24.8) (width 0.4) (layer "F.Cu") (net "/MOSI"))
 (segment (start 58.75 24.8) (end 58.75 25) (width 0.4) (layer "F.Cu") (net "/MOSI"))
 (segment (start 75.427622 28.75) (end 71.477622 24.8) (width 0.4) (layer "F.Cu") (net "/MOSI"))
 (segment (start 58.75 25) (end 44 39.75) (width 0.4) (layer "F.Cu") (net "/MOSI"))
 (segment (start 58.75 24.8) (end 58.46 24.8) (width 0.4) (layer "F.Cu") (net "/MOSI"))
 (segment (start 44 39.26) (end 58.46 24.8) (width 0.3) (layer "F.Cu") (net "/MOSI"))
 (segment (start 44 41.62) (end 44 39.26) (width 0.3) (layer "F.Cu") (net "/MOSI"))
 (segment (start 76.225 28.75) (end 75.427622 28.75) (width 0.4) (layer "F.Cu") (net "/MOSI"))
 (segment (start 79.955455 28.2) (end 80.3 27.855456) (width 0.3) (layer "F.Cu") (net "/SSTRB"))
 (segment (start 76.225 28.1) (end 76.325 28.2) (width 0.3) (layer "F.Cu") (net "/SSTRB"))
 (segment (start 76.355456 22.7) (end 40.24 22.7) (width 0.3) (layer "F.Cu") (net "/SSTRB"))
 (segment (start 40.24 22.7) (end 38.92 24.02) (width 0.3) (layer "F.Cu") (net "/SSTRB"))
 (segment (start 76.325 28.2) (end 79.955455 28.2) (width 0.3) (layer "F.Cu") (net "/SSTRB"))
 (segment (start 38.92 24.02) (end 38.92 26.38) (width 0.3) (layer "F.Cu") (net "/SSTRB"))
 (segment (start 80.3 26.644544) (end 76.355456 22.7) (width 0.3) (layer "F.Cu") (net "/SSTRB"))
 (segment (start 80.3 27.855456) (end 80.3 26.644544) (width 0.3) (layer "F.Cu") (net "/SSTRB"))
 (segment (start 67.8 25.4) (end 61.116683 25.4) (width 0.4) (layer "F.Cu") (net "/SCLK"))
 (segment (start 61.116683 25.4) (end 45.378 41.138683) (width 0.4) (layer "F.Cu") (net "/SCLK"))
 (segment (start 45.378 41.138683) (end 45.378 42.101317) (width 0.4) (layer "F.Cu") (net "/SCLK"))
 (segment (start 45.378 42.101317) (end 46.058683 42.782) (width 0.4) (layer "F.Cu") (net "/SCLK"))
 (segment (start 46.058683 42.782) (end 47.918 42.782) (width 0.4) (layer "F.Cu") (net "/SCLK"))
 (segment (start 70.5 28.1) (end 67.8 25.4) (width 0.4) (layer "F.Cu") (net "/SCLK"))
 (segment (start 47.918 42.782) (end 49.08 41.62) (width 0.4) (layer "F.Cu") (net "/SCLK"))
 (segment (start 70.15 28.75) (end 70.1 28.7) (width 0.4) (layer "F.Cu") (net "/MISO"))
 (segment (start 64.5 26.2) (end 63.036683 26.2) (width 0.4) (layer "F.Cu") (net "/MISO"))
 (segment (start 69.652622 28.7) (end 69.3625 28.409878) (width 0.4) (layer "F.Cu") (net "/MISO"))
 (segment (start 69.3625 28.409878) (end 69.3625 27.9625) (width 0.4) (layer "F.Cu") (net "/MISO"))
 (segment (start 70.1 28.7) (end 69.652622 28.7) (width 0.4) (layer "F.Cu") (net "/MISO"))
 (segment (start 67.6 26.2) (end 64.5 26.2) (width 0.4) (layer "F.Cu") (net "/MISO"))
 (segment (start 69.3625 27.9625) (end 67.6 26.2) (width 0.4) (layer "F.Cu") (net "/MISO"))
 (segment (start 64.5 26.2) (end 61.96 26.2) (width 0.4) (layer "F.Cu") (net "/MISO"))
 (segment (start 70.5 28.75) (end 70.15 28.75) (width 0.4) (layer "F.Cu") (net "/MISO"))
 (segment (start 61.96 26.2) (end 46.54 41.62) (width 0.4) (layer "F.Cu") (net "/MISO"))
 (segment (start 61.96 26.2) (end 63.036683 26.2) (width 0.3) (layer "F.Cu") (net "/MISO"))
 (segment (start 67.825 33) (end 68.825 32) (width 0.4) (layer "F.Cu") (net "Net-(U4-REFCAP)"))
 (segment (start 68.825 32) (end 70.5 32) (width 0.4) (layer "F.Cu") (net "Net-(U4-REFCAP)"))
 (segment (start 69.3625 33.40625) (end 69.3625 32.990122) (width 0.4) (layer "F.Cu") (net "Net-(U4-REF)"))
 (segment (start 69.702622 32.65) (end 70.5 32.65) (width 0.4) (layer "F.Cu") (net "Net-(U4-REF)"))
 (segment (start 67.7875 35) (end 67.7875 34.98125) (width 0.4) (layer "F.Cu") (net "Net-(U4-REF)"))
 (segment (start 67.7875 34.98125) (end 69.3625 33.40625) (width 0.4) (layer "F.Cu") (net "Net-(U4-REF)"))
 (segment (start 69.3625 32.990122) (end 69.702622 32.65) (width 0.4) (layer "F.Cu") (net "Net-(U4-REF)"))
 (segment (start 41.01 46.25) (end 57.6875 46.25) (width 0.3) (layer "F.Cu") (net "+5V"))
 (segment (start 57.6875 46.25) (end 59.5375 44.4) (width 0.3) (layer "F.Cu") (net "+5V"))
 (segment (start 36.38 41.62) (end 41.01 46.25) (width 0.3) (layer "F.Cu") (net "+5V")))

